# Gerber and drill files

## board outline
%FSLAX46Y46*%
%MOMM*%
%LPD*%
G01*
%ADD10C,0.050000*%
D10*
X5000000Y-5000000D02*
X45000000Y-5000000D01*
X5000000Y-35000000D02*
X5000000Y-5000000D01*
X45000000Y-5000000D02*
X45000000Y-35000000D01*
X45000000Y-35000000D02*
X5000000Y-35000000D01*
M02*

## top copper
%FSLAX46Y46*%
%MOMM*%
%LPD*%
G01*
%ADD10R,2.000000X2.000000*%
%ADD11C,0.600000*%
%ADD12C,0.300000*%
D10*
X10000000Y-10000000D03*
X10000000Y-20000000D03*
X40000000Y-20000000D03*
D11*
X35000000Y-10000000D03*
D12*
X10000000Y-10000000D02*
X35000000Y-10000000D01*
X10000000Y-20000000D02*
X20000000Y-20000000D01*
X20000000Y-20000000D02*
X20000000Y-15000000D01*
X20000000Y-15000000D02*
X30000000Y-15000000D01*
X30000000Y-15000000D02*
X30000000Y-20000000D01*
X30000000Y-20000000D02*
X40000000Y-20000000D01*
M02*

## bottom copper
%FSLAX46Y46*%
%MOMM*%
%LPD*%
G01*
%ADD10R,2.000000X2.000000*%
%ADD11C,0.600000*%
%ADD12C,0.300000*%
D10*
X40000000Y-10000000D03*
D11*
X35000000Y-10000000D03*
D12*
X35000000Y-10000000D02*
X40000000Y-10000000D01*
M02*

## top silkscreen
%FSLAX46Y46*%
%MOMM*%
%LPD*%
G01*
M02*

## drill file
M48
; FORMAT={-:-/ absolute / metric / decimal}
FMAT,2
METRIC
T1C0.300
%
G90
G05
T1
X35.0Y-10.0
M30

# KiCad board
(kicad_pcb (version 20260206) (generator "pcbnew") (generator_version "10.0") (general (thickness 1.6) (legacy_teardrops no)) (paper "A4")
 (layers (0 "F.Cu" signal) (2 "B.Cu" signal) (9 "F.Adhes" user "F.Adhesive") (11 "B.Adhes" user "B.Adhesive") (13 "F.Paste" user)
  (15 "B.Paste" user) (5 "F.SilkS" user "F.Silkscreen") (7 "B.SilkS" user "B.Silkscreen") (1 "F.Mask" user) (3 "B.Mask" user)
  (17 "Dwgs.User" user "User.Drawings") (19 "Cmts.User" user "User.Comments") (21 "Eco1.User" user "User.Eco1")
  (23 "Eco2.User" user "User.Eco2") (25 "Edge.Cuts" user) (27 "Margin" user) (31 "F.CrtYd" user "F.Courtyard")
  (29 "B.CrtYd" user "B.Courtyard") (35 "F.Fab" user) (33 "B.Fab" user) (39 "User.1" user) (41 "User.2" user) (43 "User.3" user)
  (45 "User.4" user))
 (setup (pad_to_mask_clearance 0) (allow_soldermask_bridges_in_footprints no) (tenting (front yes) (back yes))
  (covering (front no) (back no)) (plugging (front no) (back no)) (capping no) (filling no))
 (gr_line (start 5 5) (end 45 5) (stroke (width 0.05) (type default)) (layer "Edge.Cuts"))
 (gr_line (start 5 35) (end 5 5) (stroke (width 0.05) (type default)) (layer "Edge.Cuts"))
 (gr_line (start 45 5) (end 45 35) (stroke (width 0.05) (type default)) (layer "Edge.Cuts"))
 (gr_line (start 45 35) (end 5 35) (stroke (width 0.05) (type default)) (layer "Edge.Cuts"))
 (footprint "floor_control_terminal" (layer "F.Cu") (at 10 10)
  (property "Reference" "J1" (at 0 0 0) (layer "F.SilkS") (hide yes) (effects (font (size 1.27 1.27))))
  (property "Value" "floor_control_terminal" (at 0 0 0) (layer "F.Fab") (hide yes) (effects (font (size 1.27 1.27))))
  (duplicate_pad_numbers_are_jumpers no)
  (pad "1" smd rect (at 0 0) (size 2 2) (layers "F.Cu" "F.Paste" "F.Mask") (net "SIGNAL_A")))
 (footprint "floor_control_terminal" (layer "B.Cu") (at 40 10)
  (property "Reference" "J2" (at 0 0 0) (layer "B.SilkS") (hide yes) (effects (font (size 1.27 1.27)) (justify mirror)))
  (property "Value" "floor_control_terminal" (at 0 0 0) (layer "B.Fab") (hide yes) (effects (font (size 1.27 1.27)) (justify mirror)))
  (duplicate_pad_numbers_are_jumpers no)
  (pad "1" smd rect (at 0 0) (size 2 2) (layers "B.Cu" "B.Paste" "B.Mask") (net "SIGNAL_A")))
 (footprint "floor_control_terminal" (layer "F.Cu") (at 10 20)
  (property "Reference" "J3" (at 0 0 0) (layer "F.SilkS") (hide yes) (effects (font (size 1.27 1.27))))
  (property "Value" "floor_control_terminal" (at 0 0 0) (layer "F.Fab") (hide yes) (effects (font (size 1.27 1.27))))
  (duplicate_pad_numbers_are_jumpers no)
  (pad "1" smd rect (at 0 0) (size 2 2) (layers "F.Cu" "F.Paste" "F.Mask") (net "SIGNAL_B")))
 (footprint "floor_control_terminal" (layer "F.Cu") (at 40 20)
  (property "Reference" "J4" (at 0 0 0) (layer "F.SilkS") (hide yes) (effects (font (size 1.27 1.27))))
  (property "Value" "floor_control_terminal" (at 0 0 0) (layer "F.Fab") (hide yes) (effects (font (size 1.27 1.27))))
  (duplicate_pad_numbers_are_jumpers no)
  (pad "1" smd rect (at 0 0) (size 2 2) (layers "F.Cu" "F.Paste" "F.Mask") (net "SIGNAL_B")))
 (segment (start 10 10) (end 35 10) (width 0.3) (layer "F.Cu") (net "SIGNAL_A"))
 (segment (start 35 10) (end 40 10) (width 0.3) (layer "B.Cu") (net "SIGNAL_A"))
 (via (at 35 10) (size 0.6) (drill 0.3) (layers "F.Cu" "B.Cu") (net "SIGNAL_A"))
 (segment (start 10 20) (end 20 20) (width 0.3) (layer "F.Cu") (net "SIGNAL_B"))
 (segment (start 20 20) (end 20 15) (width 0.3) (layer "F.Cu") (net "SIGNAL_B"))
 (segment (start 20 15) (end 30 15) (width 0.3) (layer "F.Cu") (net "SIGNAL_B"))
 (segment (start 30 15) (end 30 20) (width 0.3) (layer "F.Cu") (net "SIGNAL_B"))
 (segment (start 30 20) (end 40 20) (width 0.3) (layer "F.Cu") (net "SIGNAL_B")))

